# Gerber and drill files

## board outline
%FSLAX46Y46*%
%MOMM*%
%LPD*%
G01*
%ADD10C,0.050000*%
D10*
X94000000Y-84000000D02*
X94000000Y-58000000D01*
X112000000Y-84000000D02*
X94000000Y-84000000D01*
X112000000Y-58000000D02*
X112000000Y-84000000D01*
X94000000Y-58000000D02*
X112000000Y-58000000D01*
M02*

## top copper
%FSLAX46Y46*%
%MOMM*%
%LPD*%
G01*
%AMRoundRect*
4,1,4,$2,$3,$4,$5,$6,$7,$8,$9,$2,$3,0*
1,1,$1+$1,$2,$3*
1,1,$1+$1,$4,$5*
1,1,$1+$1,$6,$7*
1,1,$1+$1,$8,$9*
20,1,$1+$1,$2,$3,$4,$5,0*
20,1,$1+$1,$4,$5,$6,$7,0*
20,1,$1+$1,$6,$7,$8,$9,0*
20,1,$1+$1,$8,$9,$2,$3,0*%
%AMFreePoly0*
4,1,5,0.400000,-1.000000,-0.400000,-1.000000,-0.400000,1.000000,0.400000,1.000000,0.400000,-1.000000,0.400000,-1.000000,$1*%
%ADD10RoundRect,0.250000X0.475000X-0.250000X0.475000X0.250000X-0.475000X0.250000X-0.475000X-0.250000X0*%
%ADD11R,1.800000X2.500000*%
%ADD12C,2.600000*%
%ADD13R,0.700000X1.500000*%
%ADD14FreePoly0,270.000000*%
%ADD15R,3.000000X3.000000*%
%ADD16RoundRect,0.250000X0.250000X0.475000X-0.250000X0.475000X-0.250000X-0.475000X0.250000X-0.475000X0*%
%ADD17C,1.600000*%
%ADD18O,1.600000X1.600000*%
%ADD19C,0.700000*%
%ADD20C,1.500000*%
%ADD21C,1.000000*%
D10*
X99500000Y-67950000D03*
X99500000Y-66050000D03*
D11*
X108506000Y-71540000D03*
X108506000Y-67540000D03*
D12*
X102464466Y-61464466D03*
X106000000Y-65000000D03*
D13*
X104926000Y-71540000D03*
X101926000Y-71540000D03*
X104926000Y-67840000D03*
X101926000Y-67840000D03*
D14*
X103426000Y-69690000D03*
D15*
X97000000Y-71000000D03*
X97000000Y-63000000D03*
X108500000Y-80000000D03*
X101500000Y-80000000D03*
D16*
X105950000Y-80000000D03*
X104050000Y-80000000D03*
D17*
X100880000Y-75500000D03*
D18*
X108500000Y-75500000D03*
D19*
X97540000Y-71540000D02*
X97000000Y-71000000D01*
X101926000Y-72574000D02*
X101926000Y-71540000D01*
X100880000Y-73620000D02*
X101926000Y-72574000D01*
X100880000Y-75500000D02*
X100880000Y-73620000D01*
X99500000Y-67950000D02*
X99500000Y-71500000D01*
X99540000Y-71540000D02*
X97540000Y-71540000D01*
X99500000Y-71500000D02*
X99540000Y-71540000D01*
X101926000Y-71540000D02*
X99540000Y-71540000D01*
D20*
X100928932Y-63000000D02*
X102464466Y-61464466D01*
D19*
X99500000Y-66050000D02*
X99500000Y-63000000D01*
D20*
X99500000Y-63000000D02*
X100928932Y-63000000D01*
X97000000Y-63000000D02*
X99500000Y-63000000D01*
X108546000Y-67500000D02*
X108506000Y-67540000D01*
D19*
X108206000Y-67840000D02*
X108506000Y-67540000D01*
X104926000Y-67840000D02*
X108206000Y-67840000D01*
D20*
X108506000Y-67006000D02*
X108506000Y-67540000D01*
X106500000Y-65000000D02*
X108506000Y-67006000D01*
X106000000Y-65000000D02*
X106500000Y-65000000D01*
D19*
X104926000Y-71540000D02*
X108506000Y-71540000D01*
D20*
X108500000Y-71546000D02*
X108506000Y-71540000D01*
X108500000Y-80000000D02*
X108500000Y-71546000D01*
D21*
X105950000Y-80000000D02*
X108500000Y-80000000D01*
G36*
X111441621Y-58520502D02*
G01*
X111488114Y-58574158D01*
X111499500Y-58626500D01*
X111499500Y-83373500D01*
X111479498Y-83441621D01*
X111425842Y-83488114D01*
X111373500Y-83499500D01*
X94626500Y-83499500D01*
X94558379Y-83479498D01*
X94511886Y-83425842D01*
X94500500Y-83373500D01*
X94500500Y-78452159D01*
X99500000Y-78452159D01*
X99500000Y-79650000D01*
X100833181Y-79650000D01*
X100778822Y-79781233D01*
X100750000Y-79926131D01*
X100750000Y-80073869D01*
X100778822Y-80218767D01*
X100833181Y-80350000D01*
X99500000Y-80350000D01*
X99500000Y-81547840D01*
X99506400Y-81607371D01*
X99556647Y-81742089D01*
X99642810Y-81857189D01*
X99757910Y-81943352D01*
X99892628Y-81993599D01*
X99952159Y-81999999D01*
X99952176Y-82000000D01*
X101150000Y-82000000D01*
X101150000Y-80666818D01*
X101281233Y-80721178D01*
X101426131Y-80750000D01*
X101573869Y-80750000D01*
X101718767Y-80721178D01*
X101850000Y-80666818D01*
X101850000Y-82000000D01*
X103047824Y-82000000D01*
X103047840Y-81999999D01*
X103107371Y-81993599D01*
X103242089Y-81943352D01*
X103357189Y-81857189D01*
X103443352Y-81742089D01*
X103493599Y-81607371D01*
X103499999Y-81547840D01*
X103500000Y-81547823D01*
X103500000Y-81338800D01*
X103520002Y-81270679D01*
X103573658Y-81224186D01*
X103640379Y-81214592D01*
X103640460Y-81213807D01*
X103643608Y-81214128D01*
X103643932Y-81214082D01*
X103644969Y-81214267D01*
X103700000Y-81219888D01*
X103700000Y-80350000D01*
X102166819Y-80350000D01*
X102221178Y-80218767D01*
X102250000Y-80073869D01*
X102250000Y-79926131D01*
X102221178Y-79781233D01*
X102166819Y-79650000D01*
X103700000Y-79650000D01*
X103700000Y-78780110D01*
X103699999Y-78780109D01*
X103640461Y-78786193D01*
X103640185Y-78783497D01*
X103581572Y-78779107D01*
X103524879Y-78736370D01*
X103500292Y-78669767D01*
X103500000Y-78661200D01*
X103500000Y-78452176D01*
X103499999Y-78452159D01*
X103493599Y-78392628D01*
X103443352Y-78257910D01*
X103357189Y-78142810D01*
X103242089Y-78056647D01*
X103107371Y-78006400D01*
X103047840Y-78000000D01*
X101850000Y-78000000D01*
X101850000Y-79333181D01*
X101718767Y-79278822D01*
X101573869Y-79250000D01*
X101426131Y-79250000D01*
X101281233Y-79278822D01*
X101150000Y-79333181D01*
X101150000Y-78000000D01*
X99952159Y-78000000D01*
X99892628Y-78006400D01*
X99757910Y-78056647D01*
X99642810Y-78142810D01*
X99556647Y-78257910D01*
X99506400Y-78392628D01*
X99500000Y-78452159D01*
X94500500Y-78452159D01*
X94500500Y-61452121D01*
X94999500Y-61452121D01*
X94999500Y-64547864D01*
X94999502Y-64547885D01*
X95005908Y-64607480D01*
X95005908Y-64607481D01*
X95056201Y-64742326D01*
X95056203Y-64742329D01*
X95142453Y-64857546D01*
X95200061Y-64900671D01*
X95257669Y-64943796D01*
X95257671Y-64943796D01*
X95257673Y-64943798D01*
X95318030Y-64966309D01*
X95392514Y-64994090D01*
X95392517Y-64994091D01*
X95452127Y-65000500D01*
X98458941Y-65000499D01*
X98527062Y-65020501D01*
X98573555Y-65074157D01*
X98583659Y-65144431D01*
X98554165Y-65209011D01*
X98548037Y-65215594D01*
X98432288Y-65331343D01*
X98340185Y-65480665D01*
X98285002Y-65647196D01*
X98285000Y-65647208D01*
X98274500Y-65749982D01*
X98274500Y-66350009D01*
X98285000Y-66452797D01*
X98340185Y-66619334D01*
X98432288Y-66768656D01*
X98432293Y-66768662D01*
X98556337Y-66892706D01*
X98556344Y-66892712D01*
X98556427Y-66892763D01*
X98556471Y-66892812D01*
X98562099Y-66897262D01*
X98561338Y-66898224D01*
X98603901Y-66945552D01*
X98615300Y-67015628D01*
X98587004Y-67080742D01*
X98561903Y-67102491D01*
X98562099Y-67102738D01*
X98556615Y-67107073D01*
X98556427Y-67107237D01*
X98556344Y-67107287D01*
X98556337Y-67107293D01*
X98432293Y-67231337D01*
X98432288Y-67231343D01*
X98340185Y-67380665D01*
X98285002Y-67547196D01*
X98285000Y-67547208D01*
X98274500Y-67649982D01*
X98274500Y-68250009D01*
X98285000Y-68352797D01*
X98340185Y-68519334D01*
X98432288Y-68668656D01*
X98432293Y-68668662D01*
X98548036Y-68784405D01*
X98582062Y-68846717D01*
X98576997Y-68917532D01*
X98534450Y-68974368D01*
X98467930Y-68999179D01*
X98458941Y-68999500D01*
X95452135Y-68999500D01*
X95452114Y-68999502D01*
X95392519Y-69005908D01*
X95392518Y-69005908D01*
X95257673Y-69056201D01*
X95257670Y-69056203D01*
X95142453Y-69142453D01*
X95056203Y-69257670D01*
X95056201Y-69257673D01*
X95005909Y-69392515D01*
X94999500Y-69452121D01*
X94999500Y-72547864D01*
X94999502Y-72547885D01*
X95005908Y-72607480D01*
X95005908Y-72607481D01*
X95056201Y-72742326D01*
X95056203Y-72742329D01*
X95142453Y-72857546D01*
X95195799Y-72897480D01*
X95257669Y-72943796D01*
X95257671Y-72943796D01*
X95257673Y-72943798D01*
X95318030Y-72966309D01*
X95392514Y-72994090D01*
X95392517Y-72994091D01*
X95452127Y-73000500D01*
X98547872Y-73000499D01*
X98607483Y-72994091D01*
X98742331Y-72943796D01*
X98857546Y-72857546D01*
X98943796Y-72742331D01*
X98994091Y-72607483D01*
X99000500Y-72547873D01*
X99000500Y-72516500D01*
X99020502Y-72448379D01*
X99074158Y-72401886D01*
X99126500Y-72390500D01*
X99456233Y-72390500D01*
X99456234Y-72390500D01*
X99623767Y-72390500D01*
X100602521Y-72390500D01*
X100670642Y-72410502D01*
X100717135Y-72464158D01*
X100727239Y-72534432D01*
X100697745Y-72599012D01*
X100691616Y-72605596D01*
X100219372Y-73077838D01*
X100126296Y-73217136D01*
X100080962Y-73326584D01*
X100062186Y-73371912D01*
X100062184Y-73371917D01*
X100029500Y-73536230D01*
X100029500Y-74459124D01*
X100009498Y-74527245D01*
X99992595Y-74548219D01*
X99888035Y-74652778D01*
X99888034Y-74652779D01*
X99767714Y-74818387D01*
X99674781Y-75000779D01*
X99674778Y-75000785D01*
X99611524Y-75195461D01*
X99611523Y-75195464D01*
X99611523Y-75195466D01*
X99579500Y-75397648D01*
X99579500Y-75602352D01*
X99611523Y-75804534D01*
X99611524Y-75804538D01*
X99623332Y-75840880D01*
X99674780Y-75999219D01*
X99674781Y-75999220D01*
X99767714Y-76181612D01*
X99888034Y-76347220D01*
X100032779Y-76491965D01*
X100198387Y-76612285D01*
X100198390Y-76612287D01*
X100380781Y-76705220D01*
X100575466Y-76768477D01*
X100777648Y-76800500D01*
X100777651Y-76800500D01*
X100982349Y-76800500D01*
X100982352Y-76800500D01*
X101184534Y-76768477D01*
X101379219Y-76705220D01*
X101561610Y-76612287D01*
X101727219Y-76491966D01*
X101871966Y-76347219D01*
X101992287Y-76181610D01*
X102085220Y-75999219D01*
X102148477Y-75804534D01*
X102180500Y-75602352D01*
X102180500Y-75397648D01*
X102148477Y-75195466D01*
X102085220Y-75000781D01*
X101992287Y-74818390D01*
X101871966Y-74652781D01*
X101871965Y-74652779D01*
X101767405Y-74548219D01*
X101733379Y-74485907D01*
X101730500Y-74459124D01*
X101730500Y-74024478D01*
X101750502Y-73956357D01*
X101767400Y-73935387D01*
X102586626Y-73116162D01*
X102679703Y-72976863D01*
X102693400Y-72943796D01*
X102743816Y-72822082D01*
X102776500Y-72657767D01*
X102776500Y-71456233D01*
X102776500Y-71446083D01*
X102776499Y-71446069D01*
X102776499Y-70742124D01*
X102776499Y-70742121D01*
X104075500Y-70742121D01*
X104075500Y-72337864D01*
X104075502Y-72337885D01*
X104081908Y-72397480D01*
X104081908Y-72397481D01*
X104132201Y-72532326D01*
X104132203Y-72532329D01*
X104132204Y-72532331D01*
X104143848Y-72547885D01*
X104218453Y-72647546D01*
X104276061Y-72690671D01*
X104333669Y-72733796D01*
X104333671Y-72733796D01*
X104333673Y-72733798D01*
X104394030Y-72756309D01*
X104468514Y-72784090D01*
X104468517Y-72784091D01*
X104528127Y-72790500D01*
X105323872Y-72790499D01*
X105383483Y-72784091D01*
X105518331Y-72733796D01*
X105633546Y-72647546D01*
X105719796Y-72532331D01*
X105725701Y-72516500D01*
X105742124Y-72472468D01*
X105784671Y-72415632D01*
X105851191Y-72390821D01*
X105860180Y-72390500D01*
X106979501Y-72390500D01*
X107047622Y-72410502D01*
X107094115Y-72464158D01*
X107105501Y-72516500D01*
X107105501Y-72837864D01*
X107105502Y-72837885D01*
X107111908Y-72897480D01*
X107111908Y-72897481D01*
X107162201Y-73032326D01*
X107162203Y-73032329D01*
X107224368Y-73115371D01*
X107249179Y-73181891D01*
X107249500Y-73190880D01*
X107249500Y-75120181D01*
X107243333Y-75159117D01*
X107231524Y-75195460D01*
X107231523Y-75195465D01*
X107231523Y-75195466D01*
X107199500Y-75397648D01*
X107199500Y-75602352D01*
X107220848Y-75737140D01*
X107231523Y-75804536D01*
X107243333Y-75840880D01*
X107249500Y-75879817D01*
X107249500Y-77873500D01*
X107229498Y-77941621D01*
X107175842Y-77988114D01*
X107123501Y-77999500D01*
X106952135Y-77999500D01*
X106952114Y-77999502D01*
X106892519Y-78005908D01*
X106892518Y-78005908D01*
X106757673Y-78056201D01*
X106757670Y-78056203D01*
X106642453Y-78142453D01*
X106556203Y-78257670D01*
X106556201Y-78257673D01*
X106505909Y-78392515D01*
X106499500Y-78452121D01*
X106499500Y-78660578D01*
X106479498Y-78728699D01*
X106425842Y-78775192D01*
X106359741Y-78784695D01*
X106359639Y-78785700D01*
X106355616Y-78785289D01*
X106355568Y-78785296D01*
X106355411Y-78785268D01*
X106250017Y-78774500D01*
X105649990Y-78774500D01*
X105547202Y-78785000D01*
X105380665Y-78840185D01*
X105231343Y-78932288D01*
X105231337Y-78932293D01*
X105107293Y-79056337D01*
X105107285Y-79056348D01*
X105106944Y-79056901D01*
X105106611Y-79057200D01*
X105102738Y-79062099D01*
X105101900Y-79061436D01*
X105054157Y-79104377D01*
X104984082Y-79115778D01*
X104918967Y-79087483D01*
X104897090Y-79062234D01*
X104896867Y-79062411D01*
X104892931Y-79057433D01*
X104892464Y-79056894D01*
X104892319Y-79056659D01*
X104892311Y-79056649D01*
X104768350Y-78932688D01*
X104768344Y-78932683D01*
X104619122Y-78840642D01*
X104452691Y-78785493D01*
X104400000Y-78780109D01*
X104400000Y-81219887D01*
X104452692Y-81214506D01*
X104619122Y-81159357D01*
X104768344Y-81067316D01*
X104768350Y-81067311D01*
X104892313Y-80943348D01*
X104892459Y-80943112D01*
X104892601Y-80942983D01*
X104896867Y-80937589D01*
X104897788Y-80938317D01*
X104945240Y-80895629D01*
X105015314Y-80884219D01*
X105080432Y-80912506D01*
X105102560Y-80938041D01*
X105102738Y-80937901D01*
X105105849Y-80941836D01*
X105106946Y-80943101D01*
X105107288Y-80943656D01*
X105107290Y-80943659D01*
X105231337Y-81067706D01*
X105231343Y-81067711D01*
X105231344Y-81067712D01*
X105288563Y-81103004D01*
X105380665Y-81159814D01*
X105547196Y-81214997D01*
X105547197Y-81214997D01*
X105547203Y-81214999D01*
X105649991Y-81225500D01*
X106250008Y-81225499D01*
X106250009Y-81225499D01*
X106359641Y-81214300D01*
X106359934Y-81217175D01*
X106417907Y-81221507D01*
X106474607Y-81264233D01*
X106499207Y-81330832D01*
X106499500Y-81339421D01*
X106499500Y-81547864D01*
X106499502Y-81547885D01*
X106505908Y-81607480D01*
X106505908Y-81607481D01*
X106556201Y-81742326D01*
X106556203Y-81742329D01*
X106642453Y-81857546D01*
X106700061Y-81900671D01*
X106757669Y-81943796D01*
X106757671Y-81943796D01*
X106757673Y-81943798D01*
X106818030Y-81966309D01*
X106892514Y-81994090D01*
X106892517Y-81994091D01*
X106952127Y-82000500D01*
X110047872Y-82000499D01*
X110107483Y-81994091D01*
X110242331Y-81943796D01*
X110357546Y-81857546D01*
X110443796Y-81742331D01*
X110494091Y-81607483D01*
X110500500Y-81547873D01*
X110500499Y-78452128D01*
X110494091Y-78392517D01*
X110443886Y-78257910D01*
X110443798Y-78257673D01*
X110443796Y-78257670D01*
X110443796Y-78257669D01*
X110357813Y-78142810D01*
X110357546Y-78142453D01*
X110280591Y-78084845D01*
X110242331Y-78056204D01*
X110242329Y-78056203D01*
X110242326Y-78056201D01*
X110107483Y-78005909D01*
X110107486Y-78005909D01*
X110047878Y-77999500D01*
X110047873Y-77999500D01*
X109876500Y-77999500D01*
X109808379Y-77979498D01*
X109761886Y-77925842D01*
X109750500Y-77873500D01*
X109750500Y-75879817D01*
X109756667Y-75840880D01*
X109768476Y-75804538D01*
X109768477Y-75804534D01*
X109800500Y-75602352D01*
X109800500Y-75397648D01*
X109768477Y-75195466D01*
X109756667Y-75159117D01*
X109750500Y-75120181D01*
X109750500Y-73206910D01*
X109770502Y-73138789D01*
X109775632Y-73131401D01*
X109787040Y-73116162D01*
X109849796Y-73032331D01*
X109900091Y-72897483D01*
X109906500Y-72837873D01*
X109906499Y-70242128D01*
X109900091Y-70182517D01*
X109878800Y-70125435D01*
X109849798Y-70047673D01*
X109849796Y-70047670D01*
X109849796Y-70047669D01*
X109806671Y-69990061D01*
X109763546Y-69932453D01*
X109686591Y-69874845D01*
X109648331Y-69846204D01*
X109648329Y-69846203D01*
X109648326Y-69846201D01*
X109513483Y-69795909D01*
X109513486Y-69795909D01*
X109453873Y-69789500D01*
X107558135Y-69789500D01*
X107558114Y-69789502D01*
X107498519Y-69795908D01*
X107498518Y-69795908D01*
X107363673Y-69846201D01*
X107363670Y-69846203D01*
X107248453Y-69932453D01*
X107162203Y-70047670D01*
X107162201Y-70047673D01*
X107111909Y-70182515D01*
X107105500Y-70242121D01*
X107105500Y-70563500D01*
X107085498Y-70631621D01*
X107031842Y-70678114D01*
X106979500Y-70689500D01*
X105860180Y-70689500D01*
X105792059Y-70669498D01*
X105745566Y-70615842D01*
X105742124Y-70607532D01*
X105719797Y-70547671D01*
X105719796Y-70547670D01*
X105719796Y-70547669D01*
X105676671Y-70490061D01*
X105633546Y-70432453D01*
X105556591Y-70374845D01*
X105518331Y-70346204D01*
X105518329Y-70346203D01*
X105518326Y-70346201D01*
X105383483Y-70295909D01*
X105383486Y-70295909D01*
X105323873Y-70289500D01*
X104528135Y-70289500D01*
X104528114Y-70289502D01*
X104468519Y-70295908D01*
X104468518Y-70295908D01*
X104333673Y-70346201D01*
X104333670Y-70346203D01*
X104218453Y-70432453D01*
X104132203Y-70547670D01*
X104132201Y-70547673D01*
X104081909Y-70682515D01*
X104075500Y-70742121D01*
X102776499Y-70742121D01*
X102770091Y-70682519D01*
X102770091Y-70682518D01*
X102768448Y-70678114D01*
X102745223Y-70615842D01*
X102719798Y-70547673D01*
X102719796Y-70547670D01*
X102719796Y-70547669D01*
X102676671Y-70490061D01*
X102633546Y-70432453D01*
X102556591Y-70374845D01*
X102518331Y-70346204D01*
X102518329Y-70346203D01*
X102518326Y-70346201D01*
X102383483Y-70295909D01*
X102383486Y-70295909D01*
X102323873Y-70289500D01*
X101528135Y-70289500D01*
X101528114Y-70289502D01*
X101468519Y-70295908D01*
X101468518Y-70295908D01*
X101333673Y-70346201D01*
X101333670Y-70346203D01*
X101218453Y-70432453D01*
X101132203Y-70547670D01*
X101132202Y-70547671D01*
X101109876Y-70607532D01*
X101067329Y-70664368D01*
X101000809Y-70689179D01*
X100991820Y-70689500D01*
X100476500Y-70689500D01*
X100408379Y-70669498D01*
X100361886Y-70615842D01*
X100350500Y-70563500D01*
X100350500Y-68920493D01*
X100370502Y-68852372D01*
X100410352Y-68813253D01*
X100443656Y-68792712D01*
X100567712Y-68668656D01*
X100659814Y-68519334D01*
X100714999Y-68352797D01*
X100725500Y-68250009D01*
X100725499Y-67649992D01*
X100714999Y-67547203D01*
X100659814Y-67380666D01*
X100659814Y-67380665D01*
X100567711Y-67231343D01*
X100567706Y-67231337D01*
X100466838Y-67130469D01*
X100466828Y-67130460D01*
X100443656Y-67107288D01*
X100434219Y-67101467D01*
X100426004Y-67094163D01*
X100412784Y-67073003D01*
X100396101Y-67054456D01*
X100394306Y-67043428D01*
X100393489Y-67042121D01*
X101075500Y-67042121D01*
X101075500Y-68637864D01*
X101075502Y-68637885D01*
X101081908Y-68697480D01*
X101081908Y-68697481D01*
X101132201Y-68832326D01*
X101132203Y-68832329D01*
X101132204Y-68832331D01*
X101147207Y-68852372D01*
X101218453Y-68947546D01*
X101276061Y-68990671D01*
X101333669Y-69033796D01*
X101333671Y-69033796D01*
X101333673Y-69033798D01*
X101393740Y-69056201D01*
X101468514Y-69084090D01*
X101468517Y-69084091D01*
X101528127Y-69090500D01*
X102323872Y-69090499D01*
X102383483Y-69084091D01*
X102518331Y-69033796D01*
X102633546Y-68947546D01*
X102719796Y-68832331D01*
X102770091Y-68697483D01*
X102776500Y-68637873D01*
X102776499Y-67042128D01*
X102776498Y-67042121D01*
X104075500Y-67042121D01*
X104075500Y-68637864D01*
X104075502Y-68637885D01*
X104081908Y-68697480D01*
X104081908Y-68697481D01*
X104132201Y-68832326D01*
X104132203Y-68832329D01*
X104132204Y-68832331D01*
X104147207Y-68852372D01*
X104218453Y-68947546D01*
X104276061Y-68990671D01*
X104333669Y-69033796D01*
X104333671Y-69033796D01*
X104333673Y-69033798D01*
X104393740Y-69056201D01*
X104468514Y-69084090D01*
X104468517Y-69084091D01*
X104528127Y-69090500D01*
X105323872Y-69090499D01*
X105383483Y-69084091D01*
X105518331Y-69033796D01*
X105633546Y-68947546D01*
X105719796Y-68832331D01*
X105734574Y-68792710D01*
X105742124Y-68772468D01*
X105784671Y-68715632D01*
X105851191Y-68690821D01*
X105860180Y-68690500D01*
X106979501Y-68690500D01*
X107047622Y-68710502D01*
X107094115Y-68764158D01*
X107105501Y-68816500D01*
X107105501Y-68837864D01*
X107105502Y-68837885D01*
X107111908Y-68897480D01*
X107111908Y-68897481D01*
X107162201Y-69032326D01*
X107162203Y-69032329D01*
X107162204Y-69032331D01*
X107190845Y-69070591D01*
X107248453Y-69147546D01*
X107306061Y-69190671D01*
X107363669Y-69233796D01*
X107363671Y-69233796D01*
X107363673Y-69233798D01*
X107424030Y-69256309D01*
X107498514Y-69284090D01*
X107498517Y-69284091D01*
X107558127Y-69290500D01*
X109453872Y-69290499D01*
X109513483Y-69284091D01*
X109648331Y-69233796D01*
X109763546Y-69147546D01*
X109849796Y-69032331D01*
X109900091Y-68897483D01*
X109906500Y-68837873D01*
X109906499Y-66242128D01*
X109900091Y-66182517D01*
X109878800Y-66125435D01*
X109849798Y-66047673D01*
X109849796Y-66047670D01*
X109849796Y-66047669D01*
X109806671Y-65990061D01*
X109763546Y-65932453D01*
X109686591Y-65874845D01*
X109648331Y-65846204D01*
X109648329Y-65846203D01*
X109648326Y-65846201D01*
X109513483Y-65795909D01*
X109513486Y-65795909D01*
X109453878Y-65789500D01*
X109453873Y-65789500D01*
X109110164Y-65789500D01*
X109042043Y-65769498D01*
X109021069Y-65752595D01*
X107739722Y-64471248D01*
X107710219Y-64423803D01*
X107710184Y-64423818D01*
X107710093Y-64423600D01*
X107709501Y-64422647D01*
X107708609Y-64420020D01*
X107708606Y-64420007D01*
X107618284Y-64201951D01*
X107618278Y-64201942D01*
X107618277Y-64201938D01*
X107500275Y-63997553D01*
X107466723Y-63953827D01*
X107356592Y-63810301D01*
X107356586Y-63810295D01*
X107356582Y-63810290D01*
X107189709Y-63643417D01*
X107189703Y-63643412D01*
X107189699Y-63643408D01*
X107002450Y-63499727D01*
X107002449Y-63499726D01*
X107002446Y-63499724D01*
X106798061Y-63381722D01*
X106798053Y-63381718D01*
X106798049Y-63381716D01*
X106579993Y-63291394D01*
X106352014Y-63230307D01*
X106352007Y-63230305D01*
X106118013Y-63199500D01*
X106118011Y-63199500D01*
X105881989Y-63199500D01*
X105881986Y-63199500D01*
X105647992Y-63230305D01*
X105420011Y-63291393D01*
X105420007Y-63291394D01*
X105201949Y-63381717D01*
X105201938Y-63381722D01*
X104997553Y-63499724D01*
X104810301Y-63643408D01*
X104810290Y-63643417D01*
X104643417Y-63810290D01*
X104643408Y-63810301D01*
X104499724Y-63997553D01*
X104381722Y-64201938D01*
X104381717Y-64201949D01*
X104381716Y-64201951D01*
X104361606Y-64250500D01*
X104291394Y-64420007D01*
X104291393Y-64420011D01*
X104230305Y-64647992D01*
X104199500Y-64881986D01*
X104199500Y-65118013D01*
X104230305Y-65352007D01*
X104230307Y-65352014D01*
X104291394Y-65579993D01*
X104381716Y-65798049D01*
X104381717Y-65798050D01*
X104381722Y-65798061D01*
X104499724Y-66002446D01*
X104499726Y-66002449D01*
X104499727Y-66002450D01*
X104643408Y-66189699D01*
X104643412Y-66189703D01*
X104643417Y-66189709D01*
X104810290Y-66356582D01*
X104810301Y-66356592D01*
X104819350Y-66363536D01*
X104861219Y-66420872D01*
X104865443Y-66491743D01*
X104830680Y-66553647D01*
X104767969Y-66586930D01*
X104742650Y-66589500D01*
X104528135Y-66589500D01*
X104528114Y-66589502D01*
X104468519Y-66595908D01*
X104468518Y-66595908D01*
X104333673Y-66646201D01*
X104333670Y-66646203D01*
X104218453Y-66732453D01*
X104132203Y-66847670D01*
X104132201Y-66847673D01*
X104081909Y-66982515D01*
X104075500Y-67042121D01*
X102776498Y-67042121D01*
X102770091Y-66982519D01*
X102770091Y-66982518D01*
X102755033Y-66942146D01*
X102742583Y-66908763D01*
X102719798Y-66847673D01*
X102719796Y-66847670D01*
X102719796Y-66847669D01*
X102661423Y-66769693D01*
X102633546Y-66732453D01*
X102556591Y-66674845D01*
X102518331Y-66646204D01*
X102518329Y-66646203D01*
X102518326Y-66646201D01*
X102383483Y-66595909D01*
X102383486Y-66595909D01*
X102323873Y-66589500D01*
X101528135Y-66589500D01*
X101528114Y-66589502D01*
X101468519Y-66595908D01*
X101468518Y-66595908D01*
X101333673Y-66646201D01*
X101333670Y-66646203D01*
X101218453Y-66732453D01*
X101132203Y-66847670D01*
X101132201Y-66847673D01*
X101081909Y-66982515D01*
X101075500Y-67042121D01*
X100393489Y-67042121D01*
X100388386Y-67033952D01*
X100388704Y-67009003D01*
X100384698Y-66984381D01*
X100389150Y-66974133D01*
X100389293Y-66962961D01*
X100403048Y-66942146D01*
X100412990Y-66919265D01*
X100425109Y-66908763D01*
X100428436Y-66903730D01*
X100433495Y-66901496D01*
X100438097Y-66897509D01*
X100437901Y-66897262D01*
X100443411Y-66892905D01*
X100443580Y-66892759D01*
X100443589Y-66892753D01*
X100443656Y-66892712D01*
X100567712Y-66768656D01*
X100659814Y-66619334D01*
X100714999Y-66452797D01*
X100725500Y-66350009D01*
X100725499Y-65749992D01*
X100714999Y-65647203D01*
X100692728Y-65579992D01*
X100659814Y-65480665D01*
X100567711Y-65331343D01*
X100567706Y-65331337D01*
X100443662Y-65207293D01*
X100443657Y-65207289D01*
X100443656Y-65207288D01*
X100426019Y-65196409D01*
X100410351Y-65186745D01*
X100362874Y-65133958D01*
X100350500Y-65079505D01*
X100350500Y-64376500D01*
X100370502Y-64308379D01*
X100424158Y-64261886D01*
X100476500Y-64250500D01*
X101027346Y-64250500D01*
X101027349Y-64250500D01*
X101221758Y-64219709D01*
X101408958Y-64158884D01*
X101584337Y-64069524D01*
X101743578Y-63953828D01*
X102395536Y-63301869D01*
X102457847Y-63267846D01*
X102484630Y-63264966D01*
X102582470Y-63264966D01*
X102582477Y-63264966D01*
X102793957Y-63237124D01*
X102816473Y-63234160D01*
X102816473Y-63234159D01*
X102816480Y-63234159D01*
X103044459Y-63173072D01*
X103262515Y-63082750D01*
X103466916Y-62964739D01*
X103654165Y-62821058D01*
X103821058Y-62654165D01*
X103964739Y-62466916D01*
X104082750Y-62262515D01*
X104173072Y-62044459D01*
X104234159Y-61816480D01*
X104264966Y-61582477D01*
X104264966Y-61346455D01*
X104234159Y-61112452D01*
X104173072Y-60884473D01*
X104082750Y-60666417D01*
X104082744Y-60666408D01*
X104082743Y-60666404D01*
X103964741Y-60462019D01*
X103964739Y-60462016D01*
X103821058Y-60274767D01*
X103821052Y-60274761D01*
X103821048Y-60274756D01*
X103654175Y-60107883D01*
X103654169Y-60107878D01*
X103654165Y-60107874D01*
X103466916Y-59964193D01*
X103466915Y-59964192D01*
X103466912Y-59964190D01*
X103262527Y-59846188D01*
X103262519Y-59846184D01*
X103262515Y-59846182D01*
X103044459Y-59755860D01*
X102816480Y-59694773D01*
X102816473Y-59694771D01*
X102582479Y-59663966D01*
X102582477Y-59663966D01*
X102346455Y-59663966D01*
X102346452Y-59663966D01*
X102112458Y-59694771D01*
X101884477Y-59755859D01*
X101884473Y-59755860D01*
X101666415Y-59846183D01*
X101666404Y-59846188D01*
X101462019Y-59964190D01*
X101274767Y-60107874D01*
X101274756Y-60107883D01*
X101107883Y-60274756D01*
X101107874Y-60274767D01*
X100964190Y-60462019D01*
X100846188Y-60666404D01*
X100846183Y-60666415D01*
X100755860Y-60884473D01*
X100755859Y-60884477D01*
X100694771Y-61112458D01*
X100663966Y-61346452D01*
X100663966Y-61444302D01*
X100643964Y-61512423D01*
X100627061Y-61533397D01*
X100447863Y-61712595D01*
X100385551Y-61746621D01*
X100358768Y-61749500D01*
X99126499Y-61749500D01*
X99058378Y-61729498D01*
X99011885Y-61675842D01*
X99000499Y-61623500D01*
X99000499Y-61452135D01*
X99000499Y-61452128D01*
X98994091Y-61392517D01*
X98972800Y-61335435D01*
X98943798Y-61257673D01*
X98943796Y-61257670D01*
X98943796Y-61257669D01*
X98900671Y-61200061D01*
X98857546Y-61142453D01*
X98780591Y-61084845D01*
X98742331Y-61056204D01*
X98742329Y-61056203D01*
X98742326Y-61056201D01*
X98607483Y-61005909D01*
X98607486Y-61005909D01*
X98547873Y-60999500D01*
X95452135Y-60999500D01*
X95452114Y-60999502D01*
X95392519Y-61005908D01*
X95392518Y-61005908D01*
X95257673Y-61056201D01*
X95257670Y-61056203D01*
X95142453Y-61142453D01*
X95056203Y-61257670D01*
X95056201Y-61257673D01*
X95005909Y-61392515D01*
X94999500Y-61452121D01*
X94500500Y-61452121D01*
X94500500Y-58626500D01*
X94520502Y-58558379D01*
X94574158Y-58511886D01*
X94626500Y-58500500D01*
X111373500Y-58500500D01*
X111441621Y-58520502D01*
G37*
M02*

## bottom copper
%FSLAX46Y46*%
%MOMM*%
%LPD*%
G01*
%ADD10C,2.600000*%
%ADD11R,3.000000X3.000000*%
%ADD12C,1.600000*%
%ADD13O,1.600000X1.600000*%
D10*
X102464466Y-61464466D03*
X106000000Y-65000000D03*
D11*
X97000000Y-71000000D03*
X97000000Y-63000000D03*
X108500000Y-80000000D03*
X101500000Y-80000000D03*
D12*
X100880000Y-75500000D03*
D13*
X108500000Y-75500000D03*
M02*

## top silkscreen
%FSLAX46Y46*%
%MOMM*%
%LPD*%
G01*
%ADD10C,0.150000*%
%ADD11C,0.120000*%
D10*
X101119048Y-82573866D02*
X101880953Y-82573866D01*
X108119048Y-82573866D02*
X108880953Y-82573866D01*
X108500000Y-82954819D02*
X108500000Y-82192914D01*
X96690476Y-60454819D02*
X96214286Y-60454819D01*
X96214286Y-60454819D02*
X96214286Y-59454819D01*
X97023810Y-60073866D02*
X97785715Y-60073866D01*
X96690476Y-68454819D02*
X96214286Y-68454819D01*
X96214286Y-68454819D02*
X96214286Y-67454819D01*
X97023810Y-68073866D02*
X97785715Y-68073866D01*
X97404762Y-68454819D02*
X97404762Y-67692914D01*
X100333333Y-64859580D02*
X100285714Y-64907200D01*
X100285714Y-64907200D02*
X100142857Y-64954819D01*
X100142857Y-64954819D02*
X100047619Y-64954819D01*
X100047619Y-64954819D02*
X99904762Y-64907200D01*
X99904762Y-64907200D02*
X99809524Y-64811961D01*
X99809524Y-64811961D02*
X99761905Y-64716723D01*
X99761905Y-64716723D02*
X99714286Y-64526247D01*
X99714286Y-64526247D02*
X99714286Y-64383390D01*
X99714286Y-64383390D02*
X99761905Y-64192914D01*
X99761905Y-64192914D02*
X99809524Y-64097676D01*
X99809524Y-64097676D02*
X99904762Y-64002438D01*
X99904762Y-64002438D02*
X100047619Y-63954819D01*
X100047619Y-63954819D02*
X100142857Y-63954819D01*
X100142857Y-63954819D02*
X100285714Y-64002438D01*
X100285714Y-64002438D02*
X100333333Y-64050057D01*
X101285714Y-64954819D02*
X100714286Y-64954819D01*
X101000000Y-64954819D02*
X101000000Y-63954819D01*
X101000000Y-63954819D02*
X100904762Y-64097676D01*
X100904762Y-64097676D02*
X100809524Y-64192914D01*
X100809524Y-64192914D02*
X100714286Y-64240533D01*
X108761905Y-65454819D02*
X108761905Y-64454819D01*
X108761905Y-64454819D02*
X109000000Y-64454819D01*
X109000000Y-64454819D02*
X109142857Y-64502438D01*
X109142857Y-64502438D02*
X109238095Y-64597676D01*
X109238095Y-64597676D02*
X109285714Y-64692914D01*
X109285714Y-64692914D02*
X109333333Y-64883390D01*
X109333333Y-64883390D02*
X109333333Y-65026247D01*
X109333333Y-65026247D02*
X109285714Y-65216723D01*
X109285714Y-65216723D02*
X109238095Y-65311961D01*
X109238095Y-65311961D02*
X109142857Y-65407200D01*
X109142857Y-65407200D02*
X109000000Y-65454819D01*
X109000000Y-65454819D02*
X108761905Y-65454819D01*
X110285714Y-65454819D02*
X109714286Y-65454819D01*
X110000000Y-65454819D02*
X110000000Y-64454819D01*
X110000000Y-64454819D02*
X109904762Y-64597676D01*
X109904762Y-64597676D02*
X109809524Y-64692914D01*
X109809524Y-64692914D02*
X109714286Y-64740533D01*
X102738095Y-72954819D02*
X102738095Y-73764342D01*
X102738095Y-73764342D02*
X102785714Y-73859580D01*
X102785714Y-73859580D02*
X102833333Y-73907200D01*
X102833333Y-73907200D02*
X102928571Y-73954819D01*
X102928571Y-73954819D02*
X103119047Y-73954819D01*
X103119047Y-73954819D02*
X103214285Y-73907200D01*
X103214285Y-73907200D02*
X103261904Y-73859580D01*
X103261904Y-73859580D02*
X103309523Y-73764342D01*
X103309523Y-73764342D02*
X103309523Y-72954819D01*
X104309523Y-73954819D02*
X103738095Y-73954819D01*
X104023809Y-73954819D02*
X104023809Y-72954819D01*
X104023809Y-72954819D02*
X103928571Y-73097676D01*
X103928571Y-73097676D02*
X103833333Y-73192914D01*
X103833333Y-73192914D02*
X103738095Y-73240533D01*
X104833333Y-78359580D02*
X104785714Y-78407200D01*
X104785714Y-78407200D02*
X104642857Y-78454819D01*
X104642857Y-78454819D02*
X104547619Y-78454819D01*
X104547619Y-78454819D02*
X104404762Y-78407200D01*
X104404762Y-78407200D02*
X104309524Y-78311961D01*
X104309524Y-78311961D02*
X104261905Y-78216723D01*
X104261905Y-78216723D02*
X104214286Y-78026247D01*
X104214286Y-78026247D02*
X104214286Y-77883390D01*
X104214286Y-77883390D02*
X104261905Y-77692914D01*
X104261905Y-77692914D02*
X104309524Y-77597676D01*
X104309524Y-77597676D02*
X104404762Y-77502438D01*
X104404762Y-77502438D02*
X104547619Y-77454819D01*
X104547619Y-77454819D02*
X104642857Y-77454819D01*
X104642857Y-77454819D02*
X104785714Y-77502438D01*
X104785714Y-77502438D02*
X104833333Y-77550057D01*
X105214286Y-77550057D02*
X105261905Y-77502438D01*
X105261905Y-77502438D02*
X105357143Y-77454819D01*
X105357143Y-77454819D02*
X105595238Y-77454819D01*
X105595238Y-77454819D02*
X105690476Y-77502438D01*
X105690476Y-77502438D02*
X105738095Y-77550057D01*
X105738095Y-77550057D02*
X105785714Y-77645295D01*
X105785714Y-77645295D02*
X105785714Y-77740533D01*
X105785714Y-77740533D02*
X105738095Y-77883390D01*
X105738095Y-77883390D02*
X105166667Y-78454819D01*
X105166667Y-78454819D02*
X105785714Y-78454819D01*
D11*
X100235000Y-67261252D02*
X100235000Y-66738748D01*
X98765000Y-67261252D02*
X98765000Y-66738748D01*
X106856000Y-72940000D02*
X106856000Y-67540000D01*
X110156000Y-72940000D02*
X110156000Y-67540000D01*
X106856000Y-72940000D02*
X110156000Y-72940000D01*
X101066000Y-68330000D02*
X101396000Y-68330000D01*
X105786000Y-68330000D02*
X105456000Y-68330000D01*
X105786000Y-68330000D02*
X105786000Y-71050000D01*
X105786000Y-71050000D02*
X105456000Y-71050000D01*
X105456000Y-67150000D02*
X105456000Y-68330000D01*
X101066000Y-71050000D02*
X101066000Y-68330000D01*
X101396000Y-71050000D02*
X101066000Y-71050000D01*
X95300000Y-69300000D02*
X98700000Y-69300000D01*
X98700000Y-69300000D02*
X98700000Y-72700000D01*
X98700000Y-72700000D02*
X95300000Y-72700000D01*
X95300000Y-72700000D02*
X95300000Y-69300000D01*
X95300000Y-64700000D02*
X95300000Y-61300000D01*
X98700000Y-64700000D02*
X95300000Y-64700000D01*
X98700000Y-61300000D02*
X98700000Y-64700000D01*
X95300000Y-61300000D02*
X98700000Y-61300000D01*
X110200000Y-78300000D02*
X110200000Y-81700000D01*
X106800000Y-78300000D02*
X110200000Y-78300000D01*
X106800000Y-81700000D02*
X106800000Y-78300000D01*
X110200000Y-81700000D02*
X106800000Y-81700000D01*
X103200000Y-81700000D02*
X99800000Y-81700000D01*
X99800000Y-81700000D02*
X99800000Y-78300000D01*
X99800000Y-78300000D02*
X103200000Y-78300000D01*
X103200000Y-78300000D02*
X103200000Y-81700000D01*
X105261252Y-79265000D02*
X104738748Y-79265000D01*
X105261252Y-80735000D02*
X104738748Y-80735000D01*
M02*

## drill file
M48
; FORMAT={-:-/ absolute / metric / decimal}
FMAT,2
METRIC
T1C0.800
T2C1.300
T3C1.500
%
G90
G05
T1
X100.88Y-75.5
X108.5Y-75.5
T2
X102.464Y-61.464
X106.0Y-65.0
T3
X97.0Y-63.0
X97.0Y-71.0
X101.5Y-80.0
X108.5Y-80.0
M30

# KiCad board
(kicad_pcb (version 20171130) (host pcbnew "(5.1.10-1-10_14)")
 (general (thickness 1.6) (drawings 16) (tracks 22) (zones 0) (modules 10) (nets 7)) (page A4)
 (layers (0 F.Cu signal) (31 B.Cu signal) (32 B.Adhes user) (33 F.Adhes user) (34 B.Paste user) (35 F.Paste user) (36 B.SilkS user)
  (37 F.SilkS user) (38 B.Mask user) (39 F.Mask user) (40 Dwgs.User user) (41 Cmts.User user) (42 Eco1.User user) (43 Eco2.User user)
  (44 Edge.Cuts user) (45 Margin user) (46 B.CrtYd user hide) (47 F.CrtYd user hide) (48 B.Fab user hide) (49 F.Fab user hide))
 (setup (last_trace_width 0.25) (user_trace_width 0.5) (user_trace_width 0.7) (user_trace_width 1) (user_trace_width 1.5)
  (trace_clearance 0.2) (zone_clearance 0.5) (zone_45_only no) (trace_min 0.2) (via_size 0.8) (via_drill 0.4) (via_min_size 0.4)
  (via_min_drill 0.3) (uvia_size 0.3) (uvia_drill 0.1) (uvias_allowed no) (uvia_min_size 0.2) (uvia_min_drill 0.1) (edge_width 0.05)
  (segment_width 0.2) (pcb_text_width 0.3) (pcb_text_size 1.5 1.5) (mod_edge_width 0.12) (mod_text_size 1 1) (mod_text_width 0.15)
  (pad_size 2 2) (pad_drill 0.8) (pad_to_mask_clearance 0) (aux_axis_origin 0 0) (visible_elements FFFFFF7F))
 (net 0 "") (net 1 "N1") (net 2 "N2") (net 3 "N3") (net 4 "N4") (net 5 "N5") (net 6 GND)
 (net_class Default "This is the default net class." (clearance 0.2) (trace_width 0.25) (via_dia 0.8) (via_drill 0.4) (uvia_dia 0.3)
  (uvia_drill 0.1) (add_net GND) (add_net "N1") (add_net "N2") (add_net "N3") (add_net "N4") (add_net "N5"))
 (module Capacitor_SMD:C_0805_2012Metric (layer F.Cu) (at 99.5 67 90)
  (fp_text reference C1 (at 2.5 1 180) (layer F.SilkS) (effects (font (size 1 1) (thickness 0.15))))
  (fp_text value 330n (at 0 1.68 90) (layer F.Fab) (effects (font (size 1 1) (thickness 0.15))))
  (fp_line (start -0.261252 0.735) (end 0.261252 0.735) (layer F.SilkS) (width 0.12))
  (fp_line (start -0.261252 -0.735) (end 0.261252 -0.735) (layer F.SilkS) (width 0.12))
  (pad 1 smd roundrect (at -0.95 0 90) (size 1 1.45) (layers F.Cu F.Paste F.Mask) (roundrect_rratio 0.25) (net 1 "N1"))
  (pad 2 smd roundrect (at 0.95 0 90) (size 1 1.45) (layers F.Cu F.Paste F.Mask) (roundrect_rratio 0.25) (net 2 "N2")))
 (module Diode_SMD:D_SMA (layer F.Cu) (at 108.506 69.54 90)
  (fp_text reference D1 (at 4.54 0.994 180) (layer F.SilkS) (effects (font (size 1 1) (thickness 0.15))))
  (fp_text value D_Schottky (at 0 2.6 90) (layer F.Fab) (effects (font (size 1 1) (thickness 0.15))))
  (fp_line (start -3.4 -1.65) (end 2 -1.65) (layer F.SilkS) (width 0.12))
  (fp_line (start -3.4 1.65) (end 2 1.65) (layer F.SilkS) (width 0.12))
  (fp_line (start -3.4 -1.65) (end -3.4 1.65) (layer F.SilkS) (width 0.12))
  (pad 1 smd rect (at -2 0 90) (size 2.5 1.8) (layers F.Cu F.Paste F.Mask) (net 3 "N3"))
  (pad 2 smd rect (at 2 0 90) (size 2.5 1.8) (layers F.Cu F.Paste F.Mask) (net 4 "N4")))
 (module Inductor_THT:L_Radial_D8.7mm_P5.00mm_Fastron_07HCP (layer B.Cu) (at 102.464466 61.464466 315)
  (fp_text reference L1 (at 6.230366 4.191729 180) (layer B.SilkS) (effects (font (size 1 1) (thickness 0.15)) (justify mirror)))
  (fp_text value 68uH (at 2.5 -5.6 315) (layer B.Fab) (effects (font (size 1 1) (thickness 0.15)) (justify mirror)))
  (pad 1 thru_hole circle (at 0 0 315) (size 2.6 2.6) (drill 1.3) (layers *.Cu *.Mask) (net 2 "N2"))
  (pad 2 thru_hole circle (at 5 0 315) (size 2.6 2.6) (drill 1.3) (layers *.Cu *.Mask) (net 4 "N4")))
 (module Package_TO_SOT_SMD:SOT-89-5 (layer F.Cu) (at 103.426 69.69 270)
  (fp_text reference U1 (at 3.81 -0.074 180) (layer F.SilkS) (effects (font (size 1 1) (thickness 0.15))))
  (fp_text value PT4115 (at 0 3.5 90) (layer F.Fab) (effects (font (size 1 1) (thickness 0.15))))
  (fp_line (start -1.36 2.36) (end -1.36 2.03) (layer F.SilkS) (width 0.12))
  (fp_line (start -1.36 -2.36) (end -1.36 -2.03) (layer F.SilkS) (width 0.12))
  (fp_line (start -1.36 -2.36) (end 1.36 -2.36) (layer F.SilkS) (width 0.12))
  (fp_line (start 1.36 -2.36) (end 1.36 -2.03) (layer F.SilkS) (width 0.12))
  (fp_line (start -2.54 -2.03) (end -1.36 -2.03) (layer F.SilkS) (width 0.12))
  (fp_line (start 1.36 2.36) (end -1.36 2.36) (layer F.SilkS) (width 0.12))
  (fp_line (start 1.36 2.03) (end 1.36 2.36) (layer F.SilkS) (width 0.12))
  (pad 5 smd rect (at 1.85 -1.5 270) (size 1.5 0.7) (layers F.Cu F.Paste F.Mask) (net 3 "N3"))
  (pad 4 smd rect (at 1.85 1.5 270) (size 1.5 0.7) (layers F.Cu F.Paste F.Mask) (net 1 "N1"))
  (pad 1 smd rect (at -1.85 -1.5 270) (size 1.5 0.7) (layers F.Cu F.Paste F.Mask) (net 4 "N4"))
  (pad 3 smd rect (at -1.85 1.5 270) (size 1.5 0.7) (layers F.Cu F.Paste F.Mask) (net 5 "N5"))
  (pad 2 smd custom (at 0 0 270) (size 0.8 2) (layers F.Cu F.Paste F.Mask) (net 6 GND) (zone_connect 2)
   (options (clearance outline) (anchor rect)) (primitives)))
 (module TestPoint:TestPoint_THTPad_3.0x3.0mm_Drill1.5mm (layer F.Cu) (at 97 71)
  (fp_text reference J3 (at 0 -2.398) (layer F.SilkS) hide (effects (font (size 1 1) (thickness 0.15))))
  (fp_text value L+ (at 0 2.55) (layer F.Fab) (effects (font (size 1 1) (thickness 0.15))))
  (fp_line (start -1.7 -1.7) (end 1.7 -1.7) (layer F.SilkS) (width 0.12))
  (fp_line (start 1.7 -1.7) (end 1.7 1.7) (layer F.SilkS) (width 0.12))
  (fp_line (start 1.7 1.7) (end -1.7 1.7) (layer F.SilkS) (width 0.12))
  (fp_line (start -1.7 1.7) (end -1.7 -1.7) (layer F.SilkS) (width 0.12))
  (pad 1 thru_hole rect (at 0 0) (size 3 3) (drill 1.5) (layers *.Cu *.Mask) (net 1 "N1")))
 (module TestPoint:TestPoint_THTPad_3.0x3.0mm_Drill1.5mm (layer F.Cu) (at 97 63)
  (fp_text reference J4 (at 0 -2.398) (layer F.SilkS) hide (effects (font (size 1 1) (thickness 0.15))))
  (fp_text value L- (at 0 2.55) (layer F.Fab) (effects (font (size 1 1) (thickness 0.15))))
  (fp_line (start -1.7 1.7) (end -1.7 -1.7) (layer F.SilkS) (width 0.12))
  (fp_line (start 1.7 1.7) (end -1.7 1.7) (layer F.SilkS) (width 0.12))
  (fp_line (start 1.7 -1.7) (end 1.7 1.7) (layer F.SilkS) (width 0.12))
  (fp_line (start -1.7 -1.7) (end 1.7 -1.7) (layer F.SilkS) (width 0.12))
  (pad 1 thru_hole rect (at 0 0) (size 3 3) (drill 1.5) (layers *.Cu *.Mask) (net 2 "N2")))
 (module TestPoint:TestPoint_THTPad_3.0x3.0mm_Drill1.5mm (layer F.Cu) (at 108.5 80 180)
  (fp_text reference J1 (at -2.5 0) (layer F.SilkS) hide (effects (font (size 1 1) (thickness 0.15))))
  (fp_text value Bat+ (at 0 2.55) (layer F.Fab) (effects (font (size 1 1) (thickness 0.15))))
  (fp_line (start -1.7 1.7) (end -1.7 -1.7) (layer F.SilkS) (width 0.12))
  (fp_line (start 1.7 1.7) (end -1.7 1.7) (layer F.SilkS) (width 0.12))
  (fp_line (start 1.7 -1.7) (end 1.7 1.7) (layer F.SilkS) (width 0.12))
  (fp_line (start -1.7 -1.7) (end 1.7 -1.7) (layer F.SilkS) (width 0.12))
  (pad 1 thru_hole rect (at 0 0 180) (size 3 3) (drill 1.5) (layers *.Cu *.Mask) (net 3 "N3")))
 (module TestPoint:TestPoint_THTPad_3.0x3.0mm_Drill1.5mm (layer F.Cu) (at 101.5 80 180)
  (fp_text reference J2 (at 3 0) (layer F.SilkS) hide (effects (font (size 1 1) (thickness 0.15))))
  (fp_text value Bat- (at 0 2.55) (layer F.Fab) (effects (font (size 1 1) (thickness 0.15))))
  (fp_line (start -1.7 -1.7) (end 1.7 -1.7) (layer F.SilkS) (width 0.12))
  (fp_line (start 1.7 -1.7) (end 1.7 1.7) (layer F.SilkS) (width 0.12))
  (fp_line (start 1.7 1.7) (end -1.7 1.7) (layer F.SilkS) (width 0.12))
  (fp_line (start -1.7 1.7) (end -1.7 -1.7) (layer F.SilkS) (width 0.12))
  (pad 1 thru_hole rect (at 0 0 180) (size 3 3) (drill 1.5) (layers *.Cu *.Mask) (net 6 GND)))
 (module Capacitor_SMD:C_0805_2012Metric (layer F.Cu) (at 105 80 180)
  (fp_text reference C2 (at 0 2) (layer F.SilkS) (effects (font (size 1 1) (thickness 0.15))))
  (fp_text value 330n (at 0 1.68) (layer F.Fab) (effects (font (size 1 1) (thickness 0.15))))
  (fp_line (start -0.261252 0.735) (end 0.261252 0.735) (layer F.SilkS) (width 0.12))
  (fp_line (start -0.261252 -0.735) (end 0.261252 -0.735) (layer F.SilkS) (width 0.12))
  (pad 1 smd roundrect (at -0.95 0 180) (size 1 1.45) (layers F.Cu F.Paste F.Mask) (roundrect_rratio 0.25) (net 3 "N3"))
  (pad 2 smd roundrect (at 0.95 0 180) (size 1 1.45) (layers F.Cu F.Paste F.Mask) (roundrect_rratio 0.25) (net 6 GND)))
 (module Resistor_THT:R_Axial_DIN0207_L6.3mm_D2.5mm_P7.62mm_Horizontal (layer B.Cu) (at 100.88 75.5)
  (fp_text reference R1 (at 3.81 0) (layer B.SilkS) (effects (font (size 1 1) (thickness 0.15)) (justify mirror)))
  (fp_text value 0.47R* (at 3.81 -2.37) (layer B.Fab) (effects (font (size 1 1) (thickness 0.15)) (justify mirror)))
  (pad 1 thru_hole circle (at 0 0) (size 1.6 1.6) (drill 0.8) (layers *.Cu *.Mask) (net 1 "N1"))
  (pad 2 thru_hole oval (at 7.62 0) (size 1.6 1.6) (drill 0.8) (layers *.Cu *.Mask) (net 3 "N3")))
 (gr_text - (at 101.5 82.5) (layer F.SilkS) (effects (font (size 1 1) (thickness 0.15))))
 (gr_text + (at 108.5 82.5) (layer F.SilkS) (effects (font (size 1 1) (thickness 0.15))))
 (gr_line (start 94 84) (end 94 58) (layer Edge.Cuts) (width 0.05))
 (gr_line (start 112 84) (end 94 84) (layer Edge.Cuts) (width 0.05))
 (gr_line (start 112 58) (end 112 84) (layer Edge.Cuts) (width 0.05))
 (gr_line (start 94 58) (end 112 58) (layer Edge.Cuts) (width 0.05))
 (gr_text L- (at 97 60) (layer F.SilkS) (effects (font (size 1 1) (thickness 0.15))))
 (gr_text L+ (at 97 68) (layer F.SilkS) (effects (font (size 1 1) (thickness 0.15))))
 (segment (start 97.54 71.54) (end 97 71) (width 0.7) (layer F.Cu) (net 1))
 (segment (start 101.926 72.574) (end 101.926 71.54) (width 0.7) (layer F.Cu) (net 1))
 (segment (start 100.88 73.62) (end 101.926 72.574) (width 0.7) (layer F.Cu) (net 1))
 (segment (start 100.88 75.5) (end 100.88 73.62) (width 0.7) (layer F.Cu) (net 1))
 (segment (start 99.5 67.95) (end 99.5 71.5) (width 0.7) (layer F.Cu) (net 1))
 (segment (start 99.54 71.54) (end 97.54 71.54) (width 0.7) (layer F.Cu) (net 1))
 (segment (start 99.5 71.5) (end 99.54 71.54) (width 0.7) (layer F.Cu) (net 1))
 (segment (start 101.926 71.54) (end 99.54 71.54) (width 0.7) (layer F.Cu) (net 1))
 (segment (start 100.928932 63) (end 102.464466 61.464466) (width 1.5) (layer F.Cu) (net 2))
 (segment (start 99.5 66.05) (end 99.5 63) (width 0.7) (layer F.Cu) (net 2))
 (segment (start 99.5 63) (end 100.928932 63) (width 1.5) (layer F.Cu) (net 2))
 (segment (start 97 63) (end 99.5 63) (width 1.5) (layer F.Cu) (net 2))
 (segment (start 108.546 67.5) (end 108.506 67.54) (width 1.5) (layer F.Cu) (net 4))
 (segment (start 108.206 67.84) (end 108.506 67.54) (width 0.7) (layer F.Cu) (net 4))
 (segment (start 104.926 67.84) (end 108.206 67.84) (width 0.7) (layer F.Cu) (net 4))
 (segment (start 108.506 67.006) (end 108.506 67.54) (width 1.5) (layer F.Cu) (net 4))
 (segment (start 106.5 65) (end 108.506 67.006) (width 1.5) (layer F.Cu) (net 4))
 (segment (start 106 65) (end 106.5 65) (width 1.5) (layer F.Cu) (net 4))
 (segment (start 104.926 71.54) (end 108.506 71.54) (width 0.7) (layer F.Cu) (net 3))
 (segment (start 108.5 71.546) (end 108.506 71.54) (width 1.5) (layer F.Cu) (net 3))
 (segment (start 108.5 80) (end 108.5 71.546) (width 1.5) (layer F.Cu) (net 3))
 (segment (start 105.95 80) (end 108.5 80) (width 1) (layer F.Cu) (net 3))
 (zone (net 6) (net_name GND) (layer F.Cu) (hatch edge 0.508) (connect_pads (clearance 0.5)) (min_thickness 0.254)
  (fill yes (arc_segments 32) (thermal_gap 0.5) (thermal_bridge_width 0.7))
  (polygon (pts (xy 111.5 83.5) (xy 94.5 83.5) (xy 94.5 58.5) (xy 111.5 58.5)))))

